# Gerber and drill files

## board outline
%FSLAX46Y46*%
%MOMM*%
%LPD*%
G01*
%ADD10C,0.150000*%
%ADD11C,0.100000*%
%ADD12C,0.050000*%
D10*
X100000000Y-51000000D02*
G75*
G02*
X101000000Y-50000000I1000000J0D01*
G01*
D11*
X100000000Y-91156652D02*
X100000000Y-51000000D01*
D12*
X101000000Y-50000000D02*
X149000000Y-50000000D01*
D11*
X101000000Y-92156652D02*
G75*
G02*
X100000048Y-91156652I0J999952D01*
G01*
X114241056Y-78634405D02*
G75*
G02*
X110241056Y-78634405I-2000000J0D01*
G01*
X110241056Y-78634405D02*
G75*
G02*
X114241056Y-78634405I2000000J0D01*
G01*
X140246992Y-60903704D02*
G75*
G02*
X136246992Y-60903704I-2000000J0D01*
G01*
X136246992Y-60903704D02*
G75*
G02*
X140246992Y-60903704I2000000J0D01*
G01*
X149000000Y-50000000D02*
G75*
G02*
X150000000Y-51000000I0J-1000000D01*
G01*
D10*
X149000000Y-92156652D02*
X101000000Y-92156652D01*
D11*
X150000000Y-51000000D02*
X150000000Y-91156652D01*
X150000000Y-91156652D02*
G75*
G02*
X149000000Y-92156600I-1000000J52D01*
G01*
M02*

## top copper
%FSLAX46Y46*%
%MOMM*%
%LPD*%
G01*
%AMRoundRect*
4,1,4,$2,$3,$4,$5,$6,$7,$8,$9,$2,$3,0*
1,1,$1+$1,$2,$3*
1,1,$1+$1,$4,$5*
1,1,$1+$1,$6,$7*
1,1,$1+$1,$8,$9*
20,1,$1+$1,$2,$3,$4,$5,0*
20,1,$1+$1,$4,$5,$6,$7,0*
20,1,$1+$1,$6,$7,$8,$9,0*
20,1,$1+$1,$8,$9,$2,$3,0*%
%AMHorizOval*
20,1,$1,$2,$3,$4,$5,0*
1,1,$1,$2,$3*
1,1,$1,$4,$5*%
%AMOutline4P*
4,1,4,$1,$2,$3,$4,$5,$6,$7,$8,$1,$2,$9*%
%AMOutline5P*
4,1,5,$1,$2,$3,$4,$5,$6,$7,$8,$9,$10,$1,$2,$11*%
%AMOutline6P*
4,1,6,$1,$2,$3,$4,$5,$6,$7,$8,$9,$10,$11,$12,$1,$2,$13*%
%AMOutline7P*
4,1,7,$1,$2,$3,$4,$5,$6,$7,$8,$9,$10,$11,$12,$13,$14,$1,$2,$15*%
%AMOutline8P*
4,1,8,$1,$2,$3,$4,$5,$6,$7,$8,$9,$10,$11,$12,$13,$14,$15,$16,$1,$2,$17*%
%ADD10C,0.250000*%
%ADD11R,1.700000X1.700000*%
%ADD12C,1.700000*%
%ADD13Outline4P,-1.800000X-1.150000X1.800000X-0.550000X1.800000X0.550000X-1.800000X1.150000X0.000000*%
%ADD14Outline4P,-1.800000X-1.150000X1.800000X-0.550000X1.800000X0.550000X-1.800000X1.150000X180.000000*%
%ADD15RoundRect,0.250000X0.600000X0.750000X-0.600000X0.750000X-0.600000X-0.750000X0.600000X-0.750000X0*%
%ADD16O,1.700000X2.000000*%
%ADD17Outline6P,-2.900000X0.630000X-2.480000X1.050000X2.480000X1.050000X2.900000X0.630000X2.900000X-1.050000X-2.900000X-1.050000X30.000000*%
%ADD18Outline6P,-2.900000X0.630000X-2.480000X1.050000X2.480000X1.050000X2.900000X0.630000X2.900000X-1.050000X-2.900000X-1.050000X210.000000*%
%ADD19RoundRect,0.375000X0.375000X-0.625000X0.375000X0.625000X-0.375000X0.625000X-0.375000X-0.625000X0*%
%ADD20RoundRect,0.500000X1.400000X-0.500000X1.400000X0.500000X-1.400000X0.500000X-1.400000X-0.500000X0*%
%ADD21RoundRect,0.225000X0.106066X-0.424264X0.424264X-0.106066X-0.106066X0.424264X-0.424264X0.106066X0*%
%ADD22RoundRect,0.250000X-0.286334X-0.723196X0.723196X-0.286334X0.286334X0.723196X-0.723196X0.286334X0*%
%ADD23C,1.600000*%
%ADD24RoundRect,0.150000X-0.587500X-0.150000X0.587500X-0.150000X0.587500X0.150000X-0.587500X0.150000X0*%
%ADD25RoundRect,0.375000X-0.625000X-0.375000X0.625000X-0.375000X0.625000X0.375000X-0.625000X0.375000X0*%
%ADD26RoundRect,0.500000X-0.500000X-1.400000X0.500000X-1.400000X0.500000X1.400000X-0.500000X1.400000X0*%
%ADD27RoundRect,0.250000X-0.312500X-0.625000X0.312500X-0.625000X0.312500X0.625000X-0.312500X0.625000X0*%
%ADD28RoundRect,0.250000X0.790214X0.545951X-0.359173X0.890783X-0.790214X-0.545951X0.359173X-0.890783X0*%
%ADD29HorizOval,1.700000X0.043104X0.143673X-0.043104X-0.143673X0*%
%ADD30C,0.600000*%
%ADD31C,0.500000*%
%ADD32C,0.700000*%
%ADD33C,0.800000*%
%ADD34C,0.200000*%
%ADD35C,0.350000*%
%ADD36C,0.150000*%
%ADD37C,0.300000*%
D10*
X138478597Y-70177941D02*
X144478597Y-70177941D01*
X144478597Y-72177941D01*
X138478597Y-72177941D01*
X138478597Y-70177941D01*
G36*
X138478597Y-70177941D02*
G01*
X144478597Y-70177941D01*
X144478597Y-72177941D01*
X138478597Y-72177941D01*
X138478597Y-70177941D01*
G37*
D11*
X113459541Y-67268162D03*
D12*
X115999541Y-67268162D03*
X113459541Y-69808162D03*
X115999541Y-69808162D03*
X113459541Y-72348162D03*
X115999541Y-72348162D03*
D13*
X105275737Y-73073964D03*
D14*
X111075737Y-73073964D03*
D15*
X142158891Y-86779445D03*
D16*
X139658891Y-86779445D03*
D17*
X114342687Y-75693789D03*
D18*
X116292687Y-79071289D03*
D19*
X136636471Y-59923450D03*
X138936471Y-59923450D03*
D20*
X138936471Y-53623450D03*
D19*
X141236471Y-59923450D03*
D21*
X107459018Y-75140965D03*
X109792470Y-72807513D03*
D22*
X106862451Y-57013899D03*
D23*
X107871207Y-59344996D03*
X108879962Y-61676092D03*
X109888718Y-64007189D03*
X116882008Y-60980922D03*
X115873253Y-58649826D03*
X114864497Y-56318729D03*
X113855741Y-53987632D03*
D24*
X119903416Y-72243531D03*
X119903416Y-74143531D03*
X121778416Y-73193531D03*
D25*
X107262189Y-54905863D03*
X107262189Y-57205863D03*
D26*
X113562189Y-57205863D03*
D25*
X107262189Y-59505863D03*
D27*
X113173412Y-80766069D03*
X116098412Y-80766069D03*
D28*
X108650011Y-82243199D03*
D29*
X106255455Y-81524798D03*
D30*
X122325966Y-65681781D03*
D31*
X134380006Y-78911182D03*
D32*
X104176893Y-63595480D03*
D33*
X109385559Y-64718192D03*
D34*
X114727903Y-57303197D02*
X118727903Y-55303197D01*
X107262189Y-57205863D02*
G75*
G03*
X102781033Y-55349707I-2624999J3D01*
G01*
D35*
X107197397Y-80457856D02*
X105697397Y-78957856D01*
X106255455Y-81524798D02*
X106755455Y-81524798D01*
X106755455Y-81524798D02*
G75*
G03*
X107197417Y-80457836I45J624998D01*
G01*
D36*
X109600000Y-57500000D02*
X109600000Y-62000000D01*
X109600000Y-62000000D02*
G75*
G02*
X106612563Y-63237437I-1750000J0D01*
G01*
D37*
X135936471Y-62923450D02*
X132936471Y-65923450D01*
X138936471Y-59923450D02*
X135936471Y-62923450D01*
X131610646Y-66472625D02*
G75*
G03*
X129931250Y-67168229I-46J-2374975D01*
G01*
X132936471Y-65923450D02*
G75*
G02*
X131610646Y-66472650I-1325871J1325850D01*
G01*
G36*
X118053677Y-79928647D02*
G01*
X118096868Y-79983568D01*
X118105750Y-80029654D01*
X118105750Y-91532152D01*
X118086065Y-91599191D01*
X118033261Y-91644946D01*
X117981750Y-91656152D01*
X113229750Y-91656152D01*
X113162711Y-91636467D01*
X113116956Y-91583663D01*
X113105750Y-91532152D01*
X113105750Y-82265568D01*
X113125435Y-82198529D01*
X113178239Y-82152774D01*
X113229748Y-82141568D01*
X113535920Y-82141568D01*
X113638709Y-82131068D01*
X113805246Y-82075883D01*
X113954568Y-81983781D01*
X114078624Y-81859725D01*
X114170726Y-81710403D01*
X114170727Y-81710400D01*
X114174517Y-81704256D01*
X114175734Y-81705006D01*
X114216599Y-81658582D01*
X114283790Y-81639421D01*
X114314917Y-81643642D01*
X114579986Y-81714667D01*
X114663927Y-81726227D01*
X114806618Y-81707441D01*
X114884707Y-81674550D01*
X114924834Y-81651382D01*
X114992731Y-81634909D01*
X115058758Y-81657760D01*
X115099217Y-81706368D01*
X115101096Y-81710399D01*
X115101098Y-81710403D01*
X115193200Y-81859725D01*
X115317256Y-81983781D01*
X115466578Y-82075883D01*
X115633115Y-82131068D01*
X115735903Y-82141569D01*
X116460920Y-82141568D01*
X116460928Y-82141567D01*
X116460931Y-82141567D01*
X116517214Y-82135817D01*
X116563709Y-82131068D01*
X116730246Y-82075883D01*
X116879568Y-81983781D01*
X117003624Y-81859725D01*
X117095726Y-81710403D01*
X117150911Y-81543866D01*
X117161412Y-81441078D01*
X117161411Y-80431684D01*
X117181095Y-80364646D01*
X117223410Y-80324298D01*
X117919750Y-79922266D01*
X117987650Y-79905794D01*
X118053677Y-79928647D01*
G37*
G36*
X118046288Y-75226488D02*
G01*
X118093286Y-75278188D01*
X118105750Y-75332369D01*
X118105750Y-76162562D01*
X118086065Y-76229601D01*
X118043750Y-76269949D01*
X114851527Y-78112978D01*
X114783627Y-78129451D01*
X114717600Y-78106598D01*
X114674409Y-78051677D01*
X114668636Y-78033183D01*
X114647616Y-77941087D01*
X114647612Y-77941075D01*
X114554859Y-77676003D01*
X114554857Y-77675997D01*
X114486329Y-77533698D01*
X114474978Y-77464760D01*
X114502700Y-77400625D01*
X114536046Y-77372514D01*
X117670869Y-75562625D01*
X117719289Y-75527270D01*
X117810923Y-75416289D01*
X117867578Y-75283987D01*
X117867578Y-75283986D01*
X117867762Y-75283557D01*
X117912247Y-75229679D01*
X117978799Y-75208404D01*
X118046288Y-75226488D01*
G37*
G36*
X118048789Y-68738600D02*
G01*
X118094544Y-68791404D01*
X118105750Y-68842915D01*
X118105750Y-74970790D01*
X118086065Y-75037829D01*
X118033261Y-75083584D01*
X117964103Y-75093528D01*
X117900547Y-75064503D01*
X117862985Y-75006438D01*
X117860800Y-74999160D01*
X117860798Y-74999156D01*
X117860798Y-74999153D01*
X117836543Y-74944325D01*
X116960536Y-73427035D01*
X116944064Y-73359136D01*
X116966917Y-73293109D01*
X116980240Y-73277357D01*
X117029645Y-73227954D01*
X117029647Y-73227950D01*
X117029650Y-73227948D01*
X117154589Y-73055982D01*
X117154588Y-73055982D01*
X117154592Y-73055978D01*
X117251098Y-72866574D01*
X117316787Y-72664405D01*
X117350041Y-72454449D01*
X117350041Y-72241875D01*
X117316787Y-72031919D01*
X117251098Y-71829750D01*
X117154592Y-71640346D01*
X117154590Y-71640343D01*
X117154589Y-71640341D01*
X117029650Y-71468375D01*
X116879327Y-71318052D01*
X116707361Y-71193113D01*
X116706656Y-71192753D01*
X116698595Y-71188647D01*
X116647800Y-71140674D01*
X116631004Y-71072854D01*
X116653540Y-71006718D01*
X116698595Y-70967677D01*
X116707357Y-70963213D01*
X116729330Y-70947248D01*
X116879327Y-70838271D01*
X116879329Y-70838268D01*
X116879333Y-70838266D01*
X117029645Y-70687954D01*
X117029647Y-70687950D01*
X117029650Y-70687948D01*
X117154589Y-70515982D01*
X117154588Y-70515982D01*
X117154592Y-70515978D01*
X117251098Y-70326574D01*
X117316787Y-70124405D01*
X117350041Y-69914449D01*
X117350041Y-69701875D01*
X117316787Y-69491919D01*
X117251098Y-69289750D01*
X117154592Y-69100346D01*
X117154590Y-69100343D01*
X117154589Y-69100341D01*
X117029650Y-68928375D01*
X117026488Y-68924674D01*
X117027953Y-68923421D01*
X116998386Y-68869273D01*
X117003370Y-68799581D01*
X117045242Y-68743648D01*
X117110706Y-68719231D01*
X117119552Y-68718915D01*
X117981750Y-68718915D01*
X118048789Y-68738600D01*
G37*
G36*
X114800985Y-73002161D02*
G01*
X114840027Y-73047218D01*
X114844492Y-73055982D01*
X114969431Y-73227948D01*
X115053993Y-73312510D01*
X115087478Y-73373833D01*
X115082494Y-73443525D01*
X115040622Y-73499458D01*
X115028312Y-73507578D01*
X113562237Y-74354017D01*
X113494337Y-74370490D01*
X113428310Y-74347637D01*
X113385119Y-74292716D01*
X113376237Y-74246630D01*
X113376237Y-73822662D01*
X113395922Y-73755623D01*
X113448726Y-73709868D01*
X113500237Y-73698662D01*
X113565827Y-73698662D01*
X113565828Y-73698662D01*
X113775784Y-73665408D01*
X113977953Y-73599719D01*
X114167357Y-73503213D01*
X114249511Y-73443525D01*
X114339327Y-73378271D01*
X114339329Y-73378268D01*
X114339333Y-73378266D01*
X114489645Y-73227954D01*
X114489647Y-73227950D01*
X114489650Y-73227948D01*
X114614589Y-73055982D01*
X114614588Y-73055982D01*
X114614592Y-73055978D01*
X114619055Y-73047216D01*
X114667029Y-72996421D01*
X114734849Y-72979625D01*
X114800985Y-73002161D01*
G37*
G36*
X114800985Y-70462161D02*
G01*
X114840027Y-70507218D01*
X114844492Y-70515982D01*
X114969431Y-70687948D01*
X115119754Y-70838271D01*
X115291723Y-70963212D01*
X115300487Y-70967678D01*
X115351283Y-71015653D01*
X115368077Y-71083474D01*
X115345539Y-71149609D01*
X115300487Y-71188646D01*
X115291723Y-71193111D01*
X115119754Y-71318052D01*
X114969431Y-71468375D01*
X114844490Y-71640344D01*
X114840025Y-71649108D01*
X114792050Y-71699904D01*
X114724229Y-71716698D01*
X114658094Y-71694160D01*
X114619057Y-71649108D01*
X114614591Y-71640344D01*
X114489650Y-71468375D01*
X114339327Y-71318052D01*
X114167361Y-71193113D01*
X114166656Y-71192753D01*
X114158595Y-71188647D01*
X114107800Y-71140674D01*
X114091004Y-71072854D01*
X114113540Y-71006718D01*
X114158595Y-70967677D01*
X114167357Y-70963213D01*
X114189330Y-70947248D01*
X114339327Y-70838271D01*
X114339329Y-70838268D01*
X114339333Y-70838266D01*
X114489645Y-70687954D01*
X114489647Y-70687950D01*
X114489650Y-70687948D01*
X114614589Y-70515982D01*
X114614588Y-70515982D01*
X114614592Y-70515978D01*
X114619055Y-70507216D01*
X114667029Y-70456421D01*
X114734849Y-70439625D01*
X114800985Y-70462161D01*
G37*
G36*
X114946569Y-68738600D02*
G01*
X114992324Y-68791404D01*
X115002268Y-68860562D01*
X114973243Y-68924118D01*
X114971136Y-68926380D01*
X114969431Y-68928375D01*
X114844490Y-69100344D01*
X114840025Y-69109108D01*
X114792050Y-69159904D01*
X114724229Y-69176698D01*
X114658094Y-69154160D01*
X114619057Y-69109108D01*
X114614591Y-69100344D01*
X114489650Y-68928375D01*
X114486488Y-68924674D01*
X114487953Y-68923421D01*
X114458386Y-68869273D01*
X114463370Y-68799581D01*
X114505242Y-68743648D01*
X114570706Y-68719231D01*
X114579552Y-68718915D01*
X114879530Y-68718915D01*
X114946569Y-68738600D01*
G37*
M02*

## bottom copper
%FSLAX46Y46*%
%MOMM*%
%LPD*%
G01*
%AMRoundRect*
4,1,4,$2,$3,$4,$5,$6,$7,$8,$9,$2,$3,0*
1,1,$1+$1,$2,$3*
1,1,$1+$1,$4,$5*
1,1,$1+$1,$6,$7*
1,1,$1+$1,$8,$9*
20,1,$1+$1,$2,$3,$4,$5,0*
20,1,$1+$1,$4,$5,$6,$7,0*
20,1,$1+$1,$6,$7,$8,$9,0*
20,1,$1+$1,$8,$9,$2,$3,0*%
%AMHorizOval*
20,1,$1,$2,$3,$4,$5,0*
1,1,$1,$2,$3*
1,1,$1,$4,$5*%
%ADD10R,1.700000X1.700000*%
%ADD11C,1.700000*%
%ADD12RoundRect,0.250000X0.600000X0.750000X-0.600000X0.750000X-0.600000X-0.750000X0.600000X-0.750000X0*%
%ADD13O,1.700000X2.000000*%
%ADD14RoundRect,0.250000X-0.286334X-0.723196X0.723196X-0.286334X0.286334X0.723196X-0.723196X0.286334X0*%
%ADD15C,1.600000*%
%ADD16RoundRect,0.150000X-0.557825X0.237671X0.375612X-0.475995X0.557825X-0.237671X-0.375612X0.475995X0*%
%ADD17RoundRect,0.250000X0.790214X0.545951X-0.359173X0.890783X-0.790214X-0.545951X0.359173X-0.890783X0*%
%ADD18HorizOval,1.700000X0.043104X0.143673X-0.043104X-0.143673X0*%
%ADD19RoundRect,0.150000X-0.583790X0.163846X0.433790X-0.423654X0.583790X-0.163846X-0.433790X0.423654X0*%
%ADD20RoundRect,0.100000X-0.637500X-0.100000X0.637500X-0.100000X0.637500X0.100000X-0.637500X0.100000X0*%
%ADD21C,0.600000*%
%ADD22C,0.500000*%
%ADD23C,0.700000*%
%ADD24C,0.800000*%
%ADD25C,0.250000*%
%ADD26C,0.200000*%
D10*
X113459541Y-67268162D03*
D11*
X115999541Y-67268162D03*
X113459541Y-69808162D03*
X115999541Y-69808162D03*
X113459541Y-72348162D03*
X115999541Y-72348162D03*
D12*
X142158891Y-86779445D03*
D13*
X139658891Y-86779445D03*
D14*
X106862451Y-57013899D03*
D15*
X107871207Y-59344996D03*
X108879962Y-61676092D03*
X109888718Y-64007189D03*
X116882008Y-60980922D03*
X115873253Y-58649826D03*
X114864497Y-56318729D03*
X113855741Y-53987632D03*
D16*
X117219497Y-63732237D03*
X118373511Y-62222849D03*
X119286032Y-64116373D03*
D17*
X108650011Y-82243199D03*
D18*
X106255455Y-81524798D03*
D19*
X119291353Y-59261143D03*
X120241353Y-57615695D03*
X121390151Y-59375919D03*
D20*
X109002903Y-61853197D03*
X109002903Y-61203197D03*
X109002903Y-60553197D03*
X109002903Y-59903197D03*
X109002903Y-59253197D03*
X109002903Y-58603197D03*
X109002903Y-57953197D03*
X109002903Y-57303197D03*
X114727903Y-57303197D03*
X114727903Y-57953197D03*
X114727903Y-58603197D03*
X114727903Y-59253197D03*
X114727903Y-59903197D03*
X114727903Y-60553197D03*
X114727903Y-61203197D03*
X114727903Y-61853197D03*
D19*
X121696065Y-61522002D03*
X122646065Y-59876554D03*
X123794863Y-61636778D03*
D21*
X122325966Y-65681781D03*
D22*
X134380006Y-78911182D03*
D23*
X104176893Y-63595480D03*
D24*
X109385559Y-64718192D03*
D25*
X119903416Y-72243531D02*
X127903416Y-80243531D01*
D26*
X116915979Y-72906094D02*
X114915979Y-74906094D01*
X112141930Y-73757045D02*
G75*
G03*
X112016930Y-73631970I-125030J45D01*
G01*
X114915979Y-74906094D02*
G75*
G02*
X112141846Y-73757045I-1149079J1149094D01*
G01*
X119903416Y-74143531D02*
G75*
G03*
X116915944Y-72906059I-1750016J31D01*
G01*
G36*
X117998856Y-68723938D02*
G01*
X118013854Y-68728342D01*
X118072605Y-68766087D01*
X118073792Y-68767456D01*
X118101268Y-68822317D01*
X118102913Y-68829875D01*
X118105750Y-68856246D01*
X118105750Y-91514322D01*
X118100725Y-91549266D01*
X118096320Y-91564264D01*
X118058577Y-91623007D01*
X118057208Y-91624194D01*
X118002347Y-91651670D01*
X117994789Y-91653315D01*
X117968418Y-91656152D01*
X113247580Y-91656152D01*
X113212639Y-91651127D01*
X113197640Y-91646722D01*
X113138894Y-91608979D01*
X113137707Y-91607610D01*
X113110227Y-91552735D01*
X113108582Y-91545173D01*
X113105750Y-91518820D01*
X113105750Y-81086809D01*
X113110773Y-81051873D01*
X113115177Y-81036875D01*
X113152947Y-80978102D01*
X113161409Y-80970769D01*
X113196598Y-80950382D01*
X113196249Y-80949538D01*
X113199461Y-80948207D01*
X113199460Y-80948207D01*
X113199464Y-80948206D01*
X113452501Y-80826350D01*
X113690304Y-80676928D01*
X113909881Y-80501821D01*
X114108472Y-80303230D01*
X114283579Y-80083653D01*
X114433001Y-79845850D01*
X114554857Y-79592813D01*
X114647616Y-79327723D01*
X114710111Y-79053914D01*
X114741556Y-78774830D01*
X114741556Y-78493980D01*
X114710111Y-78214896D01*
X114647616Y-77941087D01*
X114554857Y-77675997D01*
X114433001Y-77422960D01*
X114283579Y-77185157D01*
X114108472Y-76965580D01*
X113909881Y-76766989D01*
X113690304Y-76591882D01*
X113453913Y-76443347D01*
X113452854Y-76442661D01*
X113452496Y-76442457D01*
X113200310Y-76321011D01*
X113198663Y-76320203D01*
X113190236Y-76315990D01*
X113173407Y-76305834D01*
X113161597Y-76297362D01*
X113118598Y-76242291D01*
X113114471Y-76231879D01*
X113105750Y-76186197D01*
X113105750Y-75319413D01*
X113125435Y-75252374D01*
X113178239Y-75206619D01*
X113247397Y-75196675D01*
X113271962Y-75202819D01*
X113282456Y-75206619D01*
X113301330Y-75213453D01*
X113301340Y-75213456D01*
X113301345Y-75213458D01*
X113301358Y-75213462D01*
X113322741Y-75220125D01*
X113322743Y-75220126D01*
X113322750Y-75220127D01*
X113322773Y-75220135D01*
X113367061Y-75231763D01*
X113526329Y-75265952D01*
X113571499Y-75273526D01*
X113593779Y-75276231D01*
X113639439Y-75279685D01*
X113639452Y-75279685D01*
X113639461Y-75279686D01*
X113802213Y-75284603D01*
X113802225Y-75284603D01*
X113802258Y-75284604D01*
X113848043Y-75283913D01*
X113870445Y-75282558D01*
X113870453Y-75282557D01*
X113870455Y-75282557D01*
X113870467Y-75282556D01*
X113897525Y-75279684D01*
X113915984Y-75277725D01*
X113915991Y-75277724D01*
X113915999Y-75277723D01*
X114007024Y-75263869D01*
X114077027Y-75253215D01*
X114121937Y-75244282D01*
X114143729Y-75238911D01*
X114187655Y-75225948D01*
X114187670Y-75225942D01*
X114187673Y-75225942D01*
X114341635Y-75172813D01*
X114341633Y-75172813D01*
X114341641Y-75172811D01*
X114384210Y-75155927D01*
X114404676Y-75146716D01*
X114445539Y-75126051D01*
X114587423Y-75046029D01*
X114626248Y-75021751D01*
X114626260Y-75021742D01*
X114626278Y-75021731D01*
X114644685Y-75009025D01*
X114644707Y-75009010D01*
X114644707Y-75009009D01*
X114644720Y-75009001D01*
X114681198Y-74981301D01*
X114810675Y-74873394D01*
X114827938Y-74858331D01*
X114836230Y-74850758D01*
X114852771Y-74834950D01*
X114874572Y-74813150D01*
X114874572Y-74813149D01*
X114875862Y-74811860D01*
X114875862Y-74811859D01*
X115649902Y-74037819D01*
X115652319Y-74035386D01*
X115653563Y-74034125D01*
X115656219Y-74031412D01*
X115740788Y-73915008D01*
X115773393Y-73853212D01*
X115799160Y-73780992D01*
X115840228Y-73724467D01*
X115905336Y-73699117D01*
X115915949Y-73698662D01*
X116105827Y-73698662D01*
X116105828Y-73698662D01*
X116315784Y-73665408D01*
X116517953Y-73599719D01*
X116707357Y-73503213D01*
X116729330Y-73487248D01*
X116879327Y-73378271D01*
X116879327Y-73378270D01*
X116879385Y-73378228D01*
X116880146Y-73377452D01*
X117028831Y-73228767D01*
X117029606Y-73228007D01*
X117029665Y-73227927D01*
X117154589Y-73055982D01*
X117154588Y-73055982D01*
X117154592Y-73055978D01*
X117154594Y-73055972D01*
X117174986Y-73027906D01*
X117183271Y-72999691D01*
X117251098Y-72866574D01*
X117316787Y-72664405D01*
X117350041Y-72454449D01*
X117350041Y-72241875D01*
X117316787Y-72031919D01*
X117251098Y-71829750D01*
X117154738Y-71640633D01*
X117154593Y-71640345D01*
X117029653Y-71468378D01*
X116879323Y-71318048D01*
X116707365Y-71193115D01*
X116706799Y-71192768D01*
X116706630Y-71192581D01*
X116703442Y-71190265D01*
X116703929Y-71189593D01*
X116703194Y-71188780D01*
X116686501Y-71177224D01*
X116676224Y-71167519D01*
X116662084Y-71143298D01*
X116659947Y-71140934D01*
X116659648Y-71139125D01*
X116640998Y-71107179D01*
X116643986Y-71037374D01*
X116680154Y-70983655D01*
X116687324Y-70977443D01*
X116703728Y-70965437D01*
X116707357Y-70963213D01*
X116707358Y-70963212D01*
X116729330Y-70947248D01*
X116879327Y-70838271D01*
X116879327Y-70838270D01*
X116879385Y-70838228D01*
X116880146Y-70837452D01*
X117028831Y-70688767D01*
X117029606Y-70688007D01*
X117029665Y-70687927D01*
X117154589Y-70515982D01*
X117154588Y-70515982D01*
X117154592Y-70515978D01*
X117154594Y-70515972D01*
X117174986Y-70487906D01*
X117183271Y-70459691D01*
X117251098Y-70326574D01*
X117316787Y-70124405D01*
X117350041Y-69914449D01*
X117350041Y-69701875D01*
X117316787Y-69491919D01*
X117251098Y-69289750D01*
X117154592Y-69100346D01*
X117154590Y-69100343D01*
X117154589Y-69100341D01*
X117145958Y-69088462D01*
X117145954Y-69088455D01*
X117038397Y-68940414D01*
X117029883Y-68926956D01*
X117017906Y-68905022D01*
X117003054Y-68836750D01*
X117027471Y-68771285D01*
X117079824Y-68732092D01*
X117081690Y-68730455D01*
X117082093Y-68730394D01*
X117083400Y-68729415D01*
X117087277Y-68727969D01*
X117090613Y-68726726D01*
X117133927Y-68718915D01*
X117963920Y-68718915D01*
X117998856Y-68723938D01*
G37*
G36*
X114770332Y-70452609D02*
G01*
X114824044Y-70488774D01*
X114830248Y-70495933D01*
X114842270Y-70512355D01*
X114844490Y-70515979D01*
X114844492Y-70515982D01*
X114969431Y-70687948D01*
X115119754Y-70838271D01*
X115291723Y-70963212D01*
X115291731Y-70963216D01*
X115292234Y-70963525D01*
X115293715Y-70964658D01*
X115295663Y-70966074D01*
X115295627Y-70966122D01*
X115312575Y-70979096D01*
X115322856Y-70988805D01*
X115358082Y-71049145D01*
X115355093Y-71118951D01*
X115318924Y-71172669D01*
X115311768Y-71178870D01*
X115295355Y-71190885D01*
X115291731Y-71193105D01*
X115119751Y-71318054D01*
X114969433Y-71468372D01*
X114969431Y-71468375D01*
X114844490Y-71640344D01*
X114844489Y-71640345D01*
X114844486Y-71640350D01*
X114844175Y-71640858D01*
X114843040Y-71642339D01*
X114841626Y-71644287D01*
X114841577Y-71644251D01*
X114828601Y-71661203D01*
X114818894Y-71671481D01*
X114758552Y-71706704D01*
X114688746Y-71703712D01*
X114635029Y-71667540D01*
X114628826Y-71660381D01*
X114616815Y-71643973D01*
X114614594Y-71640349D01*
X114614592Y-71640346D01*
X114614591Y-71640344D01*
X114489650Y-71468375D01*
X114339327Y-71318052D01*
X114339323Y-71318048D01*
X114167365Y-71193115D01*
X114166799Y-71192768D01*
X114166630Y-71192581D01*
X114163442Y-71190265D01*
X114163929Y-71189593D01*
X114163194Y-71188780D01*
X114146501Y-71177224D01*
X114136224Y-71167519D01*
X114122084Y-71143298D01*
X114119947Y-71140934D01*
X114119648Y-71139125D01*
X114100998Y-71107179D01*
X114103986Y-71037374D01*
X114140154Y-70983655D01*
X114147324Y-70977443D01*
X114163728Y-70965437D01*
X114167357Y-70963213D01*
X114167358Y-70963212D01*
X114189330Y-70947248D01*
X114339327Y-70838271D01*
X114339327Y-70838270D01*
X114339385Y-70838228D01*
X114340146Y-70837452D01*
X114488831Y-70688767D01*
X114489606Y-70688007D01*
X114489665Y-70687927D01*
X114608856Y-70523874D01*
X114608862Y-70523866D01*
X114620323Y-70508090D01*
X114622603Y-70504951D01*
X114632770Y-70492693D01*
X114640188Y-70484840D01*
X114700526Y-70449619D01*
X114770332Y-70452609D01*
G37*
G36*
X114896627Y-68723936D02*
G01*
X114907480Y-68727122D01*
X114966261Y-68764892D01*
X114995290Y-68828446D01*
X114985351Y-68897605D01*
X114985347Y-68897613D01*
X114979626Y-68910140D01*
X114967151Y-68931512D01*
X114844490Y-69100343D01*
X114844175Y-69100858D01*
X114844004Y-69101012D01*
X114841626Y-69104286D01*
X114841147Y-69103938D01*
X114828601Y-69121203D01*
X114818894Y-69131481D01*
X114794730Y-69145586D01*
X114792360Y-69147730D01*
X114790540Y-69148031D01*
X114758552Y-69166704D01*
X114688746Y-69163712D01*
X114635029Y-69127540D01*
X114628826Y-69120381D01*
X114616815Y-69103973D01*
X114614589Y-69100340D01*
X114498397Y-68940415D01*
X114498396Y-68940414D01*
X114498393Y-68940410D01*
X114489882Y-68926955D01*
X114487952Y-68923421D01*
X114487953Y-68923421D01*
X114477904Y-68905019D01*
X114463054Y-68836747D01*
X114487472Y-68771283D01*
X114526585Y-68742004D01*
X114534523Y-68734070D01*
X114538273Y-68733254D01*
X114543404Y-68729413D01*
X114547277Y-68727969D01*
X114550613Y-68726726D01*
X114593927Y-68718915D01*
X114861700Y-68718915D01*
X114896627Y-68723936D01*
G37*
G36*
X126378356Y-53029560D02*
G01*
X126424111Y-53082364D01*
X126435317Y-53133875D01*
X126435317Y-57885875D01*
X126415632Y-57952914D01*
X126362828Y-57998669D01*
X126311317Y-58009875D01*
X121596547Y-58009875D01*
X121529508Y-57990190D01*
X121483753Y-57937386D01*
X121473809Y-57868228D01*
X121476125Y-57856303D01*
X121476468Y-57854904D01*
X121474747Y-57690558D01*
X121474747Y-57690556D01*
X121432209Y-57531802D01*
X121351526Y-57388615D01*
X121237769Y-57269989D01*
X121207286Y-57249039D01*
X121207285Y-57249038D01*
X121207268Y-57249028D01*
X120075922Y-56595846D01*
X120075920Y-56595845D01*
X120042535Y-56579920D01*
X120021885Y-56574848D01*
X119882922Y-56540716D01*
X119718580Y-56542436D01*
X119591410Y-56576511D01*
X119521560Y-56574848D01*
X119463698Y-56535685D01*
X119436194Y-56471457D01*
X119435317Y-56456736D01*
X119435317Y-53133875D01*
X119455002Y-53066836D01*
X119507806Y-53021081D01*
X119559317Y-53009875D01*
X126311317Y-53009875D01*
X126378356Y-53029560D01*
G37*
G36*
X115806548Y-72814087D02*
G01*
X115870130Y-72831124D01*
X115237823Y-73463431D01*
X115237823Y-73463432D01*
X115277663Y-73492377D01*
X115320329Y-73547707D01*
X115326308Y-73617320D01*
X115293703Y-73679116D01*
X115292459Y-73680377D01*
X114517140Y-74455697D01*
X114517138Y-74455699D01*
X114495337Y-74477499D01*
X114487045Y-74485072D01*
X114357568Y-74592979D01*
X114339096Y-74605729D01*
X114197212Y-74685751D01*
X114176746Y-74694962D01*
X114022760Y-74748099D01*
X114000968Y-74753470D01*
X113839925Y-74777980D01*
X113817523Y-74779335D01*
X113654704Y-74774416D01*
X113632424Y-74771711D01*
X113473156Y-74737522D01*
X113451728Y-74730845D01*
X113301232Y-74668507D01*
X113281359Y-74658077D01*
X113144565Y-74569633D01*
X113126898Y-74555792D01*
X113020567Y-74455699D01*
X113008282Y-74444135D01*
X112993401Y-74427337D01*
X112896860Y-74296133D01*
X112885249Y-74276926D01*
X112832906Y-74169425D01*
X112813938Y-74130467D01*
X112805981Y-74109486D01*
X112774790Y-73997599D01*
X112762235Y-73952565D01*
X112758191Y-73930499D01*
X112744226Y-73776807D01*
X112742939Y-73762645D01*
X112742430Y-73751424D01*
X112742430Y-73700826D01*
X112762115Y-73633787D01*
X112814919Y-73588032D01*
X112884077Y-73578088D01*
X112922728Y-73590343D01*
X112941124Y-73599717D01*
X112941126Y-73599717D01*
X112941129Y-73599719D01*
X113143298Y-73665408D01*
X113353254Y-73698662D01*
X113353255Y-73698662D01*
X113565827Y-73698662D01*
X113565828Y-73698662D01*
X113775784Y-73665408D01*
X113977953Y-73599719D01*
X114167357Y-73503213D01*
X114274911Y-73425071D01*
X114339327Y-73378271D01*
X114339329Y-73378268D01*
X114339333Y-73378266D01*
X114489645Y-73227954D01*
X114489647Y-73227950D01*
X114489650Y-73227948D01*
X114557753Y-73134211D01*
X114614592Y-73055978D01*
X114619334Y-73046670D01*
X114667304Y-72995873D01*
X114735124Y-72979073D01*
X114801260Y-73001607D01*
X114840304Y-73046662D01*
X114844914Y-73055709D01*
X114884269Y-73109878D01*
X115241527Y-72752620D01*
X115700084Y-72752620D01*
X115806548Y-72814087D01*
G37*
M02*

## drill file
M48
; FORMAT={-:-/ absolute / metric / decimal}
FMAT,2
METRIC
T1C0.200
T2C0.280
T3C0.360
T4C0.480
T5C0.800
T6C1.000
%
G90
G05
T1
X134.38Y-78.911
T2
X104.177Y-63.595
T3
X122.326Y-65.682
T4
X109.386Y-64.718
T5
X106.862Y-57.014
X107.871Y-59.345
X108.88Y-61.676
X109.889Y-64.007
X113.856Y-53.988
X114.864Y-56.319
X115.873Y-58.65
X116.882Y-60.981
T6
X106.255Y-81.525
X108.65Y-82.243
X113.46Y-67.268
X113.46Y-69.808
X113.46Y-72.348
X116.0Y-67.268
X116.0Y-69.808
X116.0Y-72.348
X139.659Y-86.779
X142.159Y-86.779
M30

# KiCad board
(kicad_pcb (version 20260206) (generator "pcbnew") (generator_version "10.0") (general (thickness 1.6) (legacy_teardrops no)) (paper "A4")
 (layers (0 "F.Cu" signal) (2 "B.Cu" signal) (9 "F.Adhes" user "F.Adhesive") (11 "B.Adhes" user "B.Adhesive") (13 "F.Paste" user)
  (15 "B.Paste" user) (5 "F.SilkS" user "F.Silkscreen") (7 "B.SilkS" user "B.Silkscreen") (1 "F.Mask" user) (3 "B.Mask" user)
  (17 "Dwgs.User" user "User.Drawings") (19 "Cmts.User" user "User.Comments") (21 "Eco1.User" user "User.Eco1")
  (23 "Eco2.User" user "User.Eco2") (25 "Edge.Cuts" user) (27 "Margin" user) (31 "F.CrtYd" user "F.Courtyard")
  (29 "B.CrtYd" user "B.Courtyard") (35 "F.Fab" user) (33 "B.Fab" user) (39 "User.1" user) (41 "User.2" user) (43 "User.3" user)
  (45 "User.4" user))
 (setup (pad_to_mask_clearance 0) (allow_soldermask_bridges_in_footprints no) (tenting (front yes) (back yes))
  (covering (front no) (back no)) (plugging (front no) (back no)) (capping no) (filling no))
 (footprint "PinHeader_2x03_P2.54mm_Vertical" (layer "F.Cu") (at 113.459541 67.268162)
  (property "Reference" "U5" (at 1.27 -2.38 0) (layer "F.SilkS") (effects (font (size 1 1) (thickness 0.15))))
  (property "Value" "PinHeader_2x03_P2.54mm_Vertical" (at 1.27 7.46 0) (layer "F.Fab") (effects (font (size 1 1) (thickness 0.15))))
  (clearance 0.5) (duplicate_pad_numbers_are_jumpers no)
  (pad "1" thru_hole rect (at 0 0) (size 1.7 1.7) (drill 1) (layers "*.Cu" "*.Mask") (remove_unused_layers no))
  (pad "2" thru_hole circle (at 2.54 0) (size 1.7 1.7) (drill 1) (layers "*.Cu" "*.Mask") (remove_unused_layers no) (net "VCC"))
  (pad "3" thru_hole circle (at 0 2.54) (size 1.7 1.7) (drill 1) (layers "*.Cu" "*.Mask") (remove_unused_layers no) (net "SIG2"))
  (pad "4" thru_hole circle (at 2.54 2.54) (size 1.7 1.7) (drill 1) (layers "*.Cu" "*.Mask") (remove_unused_layers no))
  (pad "5" thru_hole circle (at 0 5.08) (size 1.7 1.7) (drill 1) (layers "*.Cu" "*.Mask") (remove_unused_layers no) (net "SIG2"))
  (pad "6" thru_hole circle (at 2.54 5.08) (size 1.7 1.7) (drill 1) (layers "*.Cu" "*.Mask") (remove_unused_layers no) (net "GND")))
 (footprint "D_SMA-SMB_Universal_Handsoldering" (layer "F.Cu") (at 108.175737 73.073964)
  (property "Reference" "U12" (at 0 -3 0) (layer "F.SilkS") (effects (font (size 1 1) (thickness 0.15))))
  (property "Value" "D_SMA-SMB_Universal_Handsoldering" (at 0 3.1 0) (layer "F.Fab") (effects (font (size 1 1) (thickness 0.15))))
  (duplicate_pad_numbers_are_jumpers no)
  (pad "1" smd trapezoid (at -2.9 0) (size 3.6 1.7) (rect_delta 0.6 0) (layers "F.Cu" "F.Mask" "F.Paste") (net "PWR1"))
  (pad "2" smd trapezoid (at 2.9 0 180) (size 3.6 1.7) (rect_delta 0.6 0) (layers "F.Cu" "F.Mask" "F.Paste") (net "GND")))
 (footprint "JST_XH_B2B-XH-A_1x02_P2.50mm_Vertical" (layer "F.Cu") (at 142.158891 86.779445 180)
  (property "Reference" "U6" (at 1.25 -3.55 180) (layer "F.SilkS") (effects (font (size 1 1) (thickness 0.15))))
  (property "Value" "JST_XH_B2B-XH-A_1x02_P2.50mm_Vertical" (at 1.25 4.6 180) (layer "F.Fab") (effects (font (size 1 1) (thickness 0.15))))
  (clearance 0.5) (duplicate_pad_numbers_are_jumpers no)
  (pad "1" thru_hole roundrect (at 0 0 180) (size 1.7 2) (drill 1) (layers "*.Cu" "*.Mask") (remove_unused_layers no)
   (roundrect_rratio 0.147059) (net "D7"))
  (pad "2" thru_hole oval (at 2.5 0 180) (size 1.7 2) (drill 1) (layers "*.Cu" "*.Mask") (remove_unused_layers no) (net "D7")))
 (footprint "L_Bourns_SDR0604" (layer "F.Cu") (at 115.317687 77.382539 30)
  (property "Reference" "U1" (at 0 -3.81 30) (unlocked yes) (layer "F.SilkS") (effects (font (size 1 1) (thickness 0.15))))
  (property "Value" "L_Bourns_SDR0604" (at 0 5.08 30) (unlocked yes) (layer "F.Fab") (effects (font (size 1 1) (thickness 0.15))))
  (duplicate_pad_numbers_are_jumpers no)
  (pad "1" smd roundrect (at 0 -1.95 30) (size 5.8 2.1) (layers "F.Cu" "F.Mask" "F.Paste") (roundrect_rratio 0) (chamfer_ratio 0.2)
   (chamfer top_left top_right) (die_length 2))
  (pad "2" smd roundrect (at 0 1.95 210) (size 5.8 2.1) (layers "F.Cu" "F.Mask" "F.Paste") (roundrect_rratio 0) (chamfer_ratio 0.2)
   (chamfer top_left top_right) (die_length 2)))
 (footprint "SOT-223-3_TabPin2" (layer "F.Cu") (at 138.936471 56.77345 90)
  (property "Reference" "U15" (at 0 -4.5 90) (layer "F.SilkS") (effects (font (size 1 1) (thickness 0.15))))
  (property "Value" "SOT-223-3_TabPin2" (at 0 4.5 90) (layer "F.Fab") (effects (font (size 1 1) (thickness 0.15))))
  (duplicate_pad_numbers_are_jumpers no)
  (pad "1" smd roundrect (at -3.15 -2.3 90) (size 2 1.5) (layers "F.Cu" "F.Mask" "F.Paste") (roundrect_rratio 0.25) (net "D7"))
  (pad "2" smd roundrect (at -3.15 0 90) (size 2 1.5) (layers "F.Cu" "F.Mask" "F.Paste") (roundrect_rratio 0.25) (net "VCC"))
  (pad "2" smd roundrect (at 3.15 0 90) (size 2 3.8) (layers "F.Cu" "F.Mask" "F.Paste") (roundrect_rratio 0.25) (clearance 0.35))
  (pad "3" smd roundrect (at -3.15 2.3 90) (size 2 1.5) (layers "F.Cu" "F.Mask" "F.Paste") (roundrect_rratio 0.25) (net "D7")))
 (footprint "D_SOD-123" (layer "F.Cu") (at 108.625744 73.974239 45)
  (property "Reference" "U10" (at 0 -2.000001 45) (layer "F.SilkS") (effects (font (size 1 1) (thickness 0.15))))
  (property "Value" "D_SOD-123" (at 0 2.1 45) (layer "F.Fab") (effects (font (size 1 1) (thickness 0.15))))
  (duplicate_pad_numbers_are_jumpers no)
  (pad "1" smd roundrect (at -1.65 0 45) (size 0.9 1.2) (layers "F.Cu" "F.Mask" "F.Paste") (roundrect_rratio 0.25) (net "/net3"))
  (pad "2" smd roundrect (at 1.65 0 45) (size 0.9 1.2) (layers "F.Cu" "F.Mask" "F.Paste") (roundrect_rratio 0.25) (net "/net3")))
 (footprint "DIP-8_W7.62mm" (layer "F.Cu") (at 106.862451 57.013899 23.4)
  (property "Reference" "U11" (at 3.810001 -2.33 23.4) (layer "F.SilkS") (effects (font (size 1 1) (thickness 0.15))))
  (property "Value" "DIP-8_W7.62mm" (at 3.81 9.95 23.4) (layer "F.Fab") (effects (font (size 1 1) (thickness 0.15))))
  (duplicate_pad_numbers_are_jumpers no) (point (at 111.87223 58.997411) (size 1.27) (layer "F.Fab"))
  (pad "1" thru_hole roundrect (at 0 0 23.4) (size 1.6 1.6) (drill 0.8) (layers "*.Cu" "*.Mask") (remove_unused_layers no)
   (roundrect_rratio 0.15625))
  (pad "2" thru_hole circle (at 0 2.54 23.4) (size 1.6 1.6) (drill 0.8) (layers "*.Cu" "*.Mask") (remove_unused_layers no) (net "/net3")
   (clearance 0.1))
  (pad "3" thru_hole circle (at 0 5.079999 23.4) (size 1.6 1.6) (drill 0.8) (layers "*.Cu" "*.Mask") (remove_unused_layers no) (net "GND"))
  (pad "4" thru_hole circle (at 0 7.62 23.4) (size 1.6 1.6) (drill 0.8) (layers "*.Cu" "*.Mask") (remove_unused_layers no))
  (pad "5" thru_hole circle (at 7.62 7.62 23.4) (size 1.6 1.6) (drill 0.8) (layers "*.Cu" "*.Mask") (remove_unused_layers no) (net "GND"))
  (pad "6" thru_hole circle (at 7.62 5.080001 23.4) (size 1.6 1.6) (drill 0.8) (layers "*.Cu" "*.Mask") (remove_unused_layers no)
   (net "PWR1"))
  (pad "7" thru_hole circle (at 7.62 2.54 23.4) (size 1.6 1.6) (drill 0.8) (layers "*.Cu" "*.Mask") (remove_unused_layers no))
  (pad "8" thru_hole circle (at 7.62 0 23.4) (size 1.6 1.6) (drill 0.8) (layers "*.Cu" "*.Mask") (remove_unused_layers no) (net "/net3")))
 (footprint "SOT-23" (layer "F.Cu") (at 120.840916 73.193531)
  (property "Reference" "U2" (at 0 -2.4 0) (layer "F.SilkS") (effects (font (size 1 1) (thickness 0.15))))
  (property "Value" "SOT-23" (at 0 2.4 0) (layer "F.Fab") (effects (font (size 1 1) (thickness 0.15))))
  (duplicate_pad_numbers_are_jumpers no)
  (pad "1" smd roundrect (at -0.9375 -0.95) (size 1.475 0.6) (layers "F.Cu" "F.Mask" "F.Paste") (roundrect_rratio 0.25) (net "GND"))
  (pad "2" smd roundrect (at -0.9375 0.95) (size 1.475 0.6) (layers "F.Cu" "F.Mask" "F.Paste") (roundrect_rratio 0.25) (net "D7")
   (clearance 0.35))
  (pad "3" smd roundrect (at 0.9375 0) (size 1.475 0.6) (layers "F.Cu" "F.Mask" "F.Paste") (roundrect_rratio 0.25) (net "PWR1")))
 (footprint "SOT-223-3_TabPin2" (layer "F.Cu") (at 110.412189 57.205863)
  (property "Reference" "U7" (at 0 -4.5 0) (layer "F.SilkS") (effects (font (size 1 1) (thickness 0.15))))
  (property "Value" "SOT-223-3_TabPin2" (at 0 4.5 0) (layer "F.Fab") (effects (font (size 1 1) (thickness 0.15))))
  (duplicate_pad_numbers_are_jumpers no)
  (pad "1" smd roundrect (at -3.15 -2.3) (size 2 1.5) (layers "F.Cu" "F.Mask" "F.Paste") (roundrect_rratio 0.25) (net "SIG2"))
  (pad "2" smd roundrect (at -3.15 0) (size 2 1.5) (layers "F.Cu" "F.Mask" "F.Paste") (roundrect_rratio 0.25) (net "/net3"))
  (pad "2" smd roundrect (at 3.15 0) (size 2 3.8) (layers "F.Cu" "F.Mask" "F.Paste") (roundrect_rratio 0.25) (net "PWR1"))
  (pad "3" smd roundrect (at -3.15 2.3) (size 2 1.5) (layers "F.Cu" "F.Mask" "F.Paste") (roundrect_rratio 0.25)))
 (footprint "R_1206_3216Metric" (layer "F.Cu") (at 114.635912 80.766069)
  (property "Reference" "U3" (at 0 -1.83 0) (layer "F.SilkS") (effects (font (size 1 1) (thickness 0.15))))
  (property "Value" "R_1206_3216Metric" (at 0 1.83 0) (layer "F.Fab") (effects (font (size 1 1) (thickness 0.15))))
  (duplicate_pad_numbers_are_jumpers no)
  (pad "1" smd roundrect (at -1.4625 0) (size 1.125 1.75) (layers "F.Cu" "F.Mask" "F.Paste") (roundrect_rratio 0.222222) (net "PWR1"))
  (pad "2" smd roundrect (at 1.4625 0) (size 1.125 1.75) (layers "F.Cu" "F.Mask" "F.Paste") (roundrect_rratio 0.222222) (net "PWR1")))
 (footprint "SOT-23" (layer "B.Cu") (at 118.541268 63.546958 -37.4)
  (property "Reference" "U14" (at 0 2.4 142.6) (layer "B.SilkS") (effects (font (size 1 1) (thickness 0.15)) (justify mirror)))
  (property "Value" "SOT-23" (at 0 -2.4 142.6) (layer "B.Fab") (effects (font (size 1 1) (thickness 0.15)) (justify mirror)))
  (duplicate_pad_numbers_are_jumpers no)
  (pad "1" smd roundrect (at -0.9375 0.95 322.6) (size 1.475 0.6) (layers "B.Cu" "B.Mask" "B.Paste") (roundrect_rratio 0.25) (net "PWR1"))
  (pad "2" smd roundrect (at -0.9375 -0.95 322.6) (size 1.475 0.6) (layers "B.Cu" "B.Mask" "B.Paste") (roundrect_rratio 0.25) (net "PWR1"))
  (pad "3" smd roundrect (at 0.9375 0 322.6) (size 1.475 0.6) (layers "B.Cu" "B.Mask" "B.Paste") (roundrect_rratio 0.25)))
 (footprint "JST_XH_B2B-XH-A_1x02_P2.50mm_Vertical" (layer "B.Cu") (at 108.650011 82.243199 163.3)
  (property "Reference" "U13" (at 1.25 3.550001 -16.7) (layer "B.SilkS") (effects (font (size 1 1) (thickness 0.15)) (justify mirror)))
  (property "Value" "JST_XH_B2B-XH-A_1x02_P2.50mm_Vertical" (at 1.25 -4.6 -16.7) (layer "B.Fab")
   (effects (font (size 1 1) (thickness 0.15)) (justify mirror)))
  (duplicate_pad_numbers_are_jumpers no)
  (pad "1" thru_hole roundrect (at 0 0 163.3) (size 1.7 2) (drill 1) (layers "*.Cu" "*.Mask") (remove_unused_layers no)
   (roundrect_rratio 0.147059) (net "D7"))
  (pad "2" thru_hole oval (at 2.5 0 163.3) (size 1.7 2) (drill 1) (layers "*.Cu" "*.Mask") (remove_unused_layers no)))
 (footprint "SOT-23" (layer "B.Cu") (at 120.578252 58.907169 -30)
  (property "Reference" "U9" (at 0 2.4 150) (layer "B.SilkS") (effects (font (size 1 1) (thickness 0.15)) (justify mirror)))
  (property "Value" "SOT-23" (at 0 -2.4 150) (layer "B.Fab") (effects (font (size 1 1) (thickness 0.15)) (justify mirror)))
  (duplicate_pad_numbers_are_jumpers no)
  (pad "1" smd roundrect (at -0.9375 0.95 330) (size 1.475 0.6) (layers "B.Cu" "B.Mask" "B.Paste") (roundrect_rratio 0.25) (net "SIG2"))
  (pad "2" smd roundrect (at -0.9375 -0.95 330) (size 1.475 0.6) (layers "B.Cu" "B.Mask" "B.Paste") (roundrect_rratio 0.25) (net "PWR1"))
  (pad "3" smd roundrect (at 0.9375 0 330) (size 1.475 0.6) (layers "B.Cu" "B.Mask" "B.Paste") (roundrect_rratio 0.25)))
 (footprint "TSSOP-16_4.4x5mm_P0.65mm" (layer "B.Cu") (at 111.865403 59.578197)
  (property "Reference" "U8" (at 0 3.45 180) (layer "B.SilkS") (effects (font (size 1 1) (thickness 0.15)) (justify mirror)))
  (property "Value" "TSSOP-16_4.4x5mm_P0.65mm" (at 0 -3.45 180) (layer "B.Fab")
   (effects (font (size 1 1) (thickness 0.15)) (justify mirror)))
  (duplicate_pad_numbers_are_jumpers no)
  (pad "1" smd roundrect (at -2.8625 2.275) (size 1.475 0.4) (layers "B.Cu" "B.Mask" "B.Paste") (roundrect_rratio 0.25) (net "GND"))
  (pad "2" smd roundrect (at -2.8625 1.625) (size 1.475 0.4) (layers "B.Cu" "B.Mask" "B.Paste") (roundrect_rratio 0.25) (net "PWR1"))
  (pad "3" smd roundrect (at -2.8625 0.975) (size 1.475 0.4) (layers "B.Cu" "B.Mask" "B.Paste") (roundrect_rratio 0.25) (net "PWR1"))
  (pad "4" smd roundrect (at -2.8625 0.325) (size 1.475 0.4) (layers "B.Cu" "B.Mask" "B.Paste") (roundrect_rratio 0.25) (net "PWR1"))
  (pad "5" smd roundrect (at -2.8625 -0.325) (size 1.475 0.4) (layers "B.Cu" "B.Mask" "B.Paste") (roundrect_rratio 0.25) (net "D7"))
  (pad "6" smd roundrect (at -2.8625 -0.975) (size 1.475 0.4) (layers "B.Cu" "B.Mask" "B.Paste") (roundrect_rratio 0.25) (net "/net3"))
  (pad "7" smd roundrect (at -2.8625 -1.625) (size 1.475 0.4) (layers "B.Cu" "B.Mask" "B.Paste") (roundrect_rratio 0.25) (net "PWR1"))
  (pad "8" smd roundrect (at -2.8625 -2.275) (size 1.475 0.4) (layers "B.Cu" "B.Mask" "B.Paste") (roundrect_rratio 0.25) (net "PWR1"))
  (pad "9" smd roundrect (at 2.8625 -2.275) (size 1.475 0.4) (layers "B.Cu" "B.Mask" "B.Paste") (roundrect_rratio 0.25) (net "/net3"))
  (pad "10" smd roundrect (at 2.8625 -1.625) (size 1.475 0.4) (layers "B.Cu" "B.Mask" "B.Paste") (roundrect_rratio 0.25) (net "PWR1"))
  (pad "11" smd roundrect (at 2.8625 -0.975) (size 1.475 0.4) (layers "B.Cu" "B.Mask" "B.Paste") (roundrect_rratio 0.25) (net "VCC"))
  (pad "12" smd roundrect (at 2.8625 -0.325) (size 1.475 0.4) (layers "B.Cu" "B.Mask" "B.Paste") (roundrect_rratio 0.25) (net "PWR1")
   (clearance 0.35))
  (pad "13" smd roundrect (at 2.8625 0.325) (size 1.475 0.4) (layers "B.Cu" "B.Mask" "B.Paste") (roundrect_rratio 0.25) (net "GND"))
  (pad "14" smd roundrect (at 2.8625 0.975) (size 1.475 0.4) (layers "B.Cu" "B.Mask" "B.Paste") (roundrect_rratio 0.25) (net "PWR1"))
  (pad "15" smd roundrect (at 2.8625 1.625) (size 1.475 0.4) (layers "B.Cu" "B.Mask" "B.Paste") (roundrect_rratio 0.25) (clearance 0.35))
  (pad "16" smd roundrect (at 2.8625 2.275) (size 1.475 0.4) (layers "B.Cu" "B.Mask" "B.Paste") (roundrect_rratio 0.25) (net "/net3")))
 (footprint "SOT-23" (layer "B.Cu") (at 122.982964 61.168028 -30)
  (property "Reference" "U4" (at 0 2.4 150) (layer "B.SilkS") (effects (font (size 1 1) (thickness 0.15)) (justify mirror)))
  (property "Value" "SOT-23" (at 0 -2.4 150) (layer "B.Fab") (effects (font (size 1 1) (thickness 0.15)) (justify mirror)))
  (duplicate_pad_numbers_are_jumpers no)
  (pad "1" smd roundrect (at -0.9375 0.95 330) (size 1.475 0.6) (layers "B.Cu" "B.Mask" "B.Paste") (roundrect_rratio 0.25))
  (pad "2" smd roundrect (at -0.9375 -0.95 330) (size 1.475 0.6) (layers "B.Cu" "B.Mask" "B.Paste") (roundrect_rratio 0.25) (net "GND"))
  (pad "3" smd roundrect (at 0.9375 0 330) (size 1.475 0.6) (layers "B.Cu" "B.Mask" "B.Paste") (roundrect_rratio 0.25) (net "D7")))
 (gr_rect (start 138.478597 70.177941) (end 144.478597 72.177941) (stroke (width 0.25) (type default)) (fill yes) (layer "F.Cu")
  (net "PWR1"))
 (gr_arc (start 100 51) (mid 100.292893 50.292893) (end 101 50) (stroke (width 0.15) (type default)) (layer "Edge.Cuts"))
 (gr_line (start 100 91.156652) (end 100 51) (stroke (width 0.1) (type default)) (layer "Edge.Cuts"))
 (gr_line (start 101 50) (end 149 50) (stroke (width 0.05) (type default)) (layer "Edge.Cuts"))
 (gr_arc (start 101 92.156652) (mid 100.292893 91.863758) (end 100 91.156652) (stroke (width 0.1) (type default)) (layer "Edge.Cuts"))
 (gr_circle (center 112.241056 78.634405) (end 114.241056 78.634405) (stroke (width 0.1) (type default)) (fill no) (layer "Edge.Cuts"))
 (gr_circle (center 138.246992 60.903704) (end 140.246992 60.903704) (stroke (width 0.1) (type default)) (fill no) (layer "Edge.Cuts"))
 (gr_arc (start 149 50) (mid 149.707106 50.292893) (end 150 51) (stroke (width 0.1) (type default)) (layer "Edge.Cuts"))
 (gr_line (start 149 92.156652) (end 101 92.156652) (stroke (width 0.15) (type default)) (layer "Edge.Cuts"))
 (gr_line (start 150 51) (end 150 91.156652) (stroke (width 0.1) (type default)) (layer "Edge.Cuts"))
 (gr_arc (start 150 91.156652) (mid 149.707106 91.863758) (end 149 92.156652) (stroke (width 0.1) (type default)) (layer "Edge.Cuts"))
 (segment (start 114.727903 57.303197) (end 118.727903 55.303197) (width 0.2) (layer "F.Cu") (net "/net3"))
 (via (at 122.325966 65.681781) (size 0.6) (drill 0.36) (layers "F.Cu" "B.Cu") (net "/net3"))
 (arc (start 107.262189 57.205863) (mid 105.641733 54.780679) (end 102.781034 55.349708) (width 0.2) (layer "F.Cu") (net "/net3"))
 (segment (start 107.197397 80.457856) (end 105.697397 78.957856) (width 0.35) (layer "F.Cu") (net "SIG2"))
 (segment (start 106.255455 81.524798) (end 106.755455 81.524798) (width 0.35) (layer "F.Cu") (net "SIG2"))
 (arc (start 106.755455 81.524798) (mid 107.33288 81.138975) (end 107.197397 80.457856) (width 0.35) (layer "F.Cu") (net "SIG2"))
 (segment (start 109.6 57.5) (end 109.6 62) (width 0.15) (layer "F.Cu") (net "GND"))
 (arc (start 109.6 62) (mid 108.519696 63.616789) (end 106.612563 63.237437) (width 0.15) (layer "F.Cu") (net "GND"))
 (segment (start 119.903416 72.243531) (end 127.903416 80.243531) (width 0.25) (layer "B.Cu") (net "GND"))
 (via (at 134.380006 78.911182) (size 0.5) (drill 0.2) (layers "F.Cu" "B.Cu") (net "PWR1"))
 (via (at 104.176893 63.59548) (size 0.7) (drill 0.28) (layers "F.Cu" "B.Cu") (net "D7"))
 (segment (start 116.915979 72.906094) (end 114.915979 74.906094) (width 0.2) (layer "B.Cu") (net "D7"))
 (arc (start 112.14193 73.757045) (mid 112.105318 73.668657) (end 112.01693 73.632045) (width 0.2) (layer "B.Cu") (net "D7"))
 (arc (start 114.915979 74.906094) (mid 113.14507 75.25835) (end 112.14193 73.757045) (width 0.2) (layer "B.Cu") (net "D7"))
 (arc (start 119.903416 74.143531) (mid 118.823112 72.526742) (end 116.915979 72.906094) (width 0.2) (layer "B.Cu") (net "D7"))
 (segment (start 135.936471 62.92345) (end 132.936471 65.92345) (width 0.3) (layer "F.Cu") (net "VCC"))
 (segment (start 138.936471 59.92345) (end 135.936471 62.92345) (width 0.3) (layer "F.Cu") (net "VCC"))
 (via (at 109.385559 64.718192) (size 0.8) (drill 0.48) (layers "F.Cu" "B.Cu") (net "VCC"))
 (arc (start 131.610646 66.472625) (mid 130.701773 66.653411) (end 129.931267 67.168246) (width 0.3) (layer "F.Cu") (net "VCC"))
 (arc (start 132.936471 65.92345) (mid 132.328177 66.329899) (end 131.610646 66.472625) (width 0.3) (locked yes) (layer "F.Cu") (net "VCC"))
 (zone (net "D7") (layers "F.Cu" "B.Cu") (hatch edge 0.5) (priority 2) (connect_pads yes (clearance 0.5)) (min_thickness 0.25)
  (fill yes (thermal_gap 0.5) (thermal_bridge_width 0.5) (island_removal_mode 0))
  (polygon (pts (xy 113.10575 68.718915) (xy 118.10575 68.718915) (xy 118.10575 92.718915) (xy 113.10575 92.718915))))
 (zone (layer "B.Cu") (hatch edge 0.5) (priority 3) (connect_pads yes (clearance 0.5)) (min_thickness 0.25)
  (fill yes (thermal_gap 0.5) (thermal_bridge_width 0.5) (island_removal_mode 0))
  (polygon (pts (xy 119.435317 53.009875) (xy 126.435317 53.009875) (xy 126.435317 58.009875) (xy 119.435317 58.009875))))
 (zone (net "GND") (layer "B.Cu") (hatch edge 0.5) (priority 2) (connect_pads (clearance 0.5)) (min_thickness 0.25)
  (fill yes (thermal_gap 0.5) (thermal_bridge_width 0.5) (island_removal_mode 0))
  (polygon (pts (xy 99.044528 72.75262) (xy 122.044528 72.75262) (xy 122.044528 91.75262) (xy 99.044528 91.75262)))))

